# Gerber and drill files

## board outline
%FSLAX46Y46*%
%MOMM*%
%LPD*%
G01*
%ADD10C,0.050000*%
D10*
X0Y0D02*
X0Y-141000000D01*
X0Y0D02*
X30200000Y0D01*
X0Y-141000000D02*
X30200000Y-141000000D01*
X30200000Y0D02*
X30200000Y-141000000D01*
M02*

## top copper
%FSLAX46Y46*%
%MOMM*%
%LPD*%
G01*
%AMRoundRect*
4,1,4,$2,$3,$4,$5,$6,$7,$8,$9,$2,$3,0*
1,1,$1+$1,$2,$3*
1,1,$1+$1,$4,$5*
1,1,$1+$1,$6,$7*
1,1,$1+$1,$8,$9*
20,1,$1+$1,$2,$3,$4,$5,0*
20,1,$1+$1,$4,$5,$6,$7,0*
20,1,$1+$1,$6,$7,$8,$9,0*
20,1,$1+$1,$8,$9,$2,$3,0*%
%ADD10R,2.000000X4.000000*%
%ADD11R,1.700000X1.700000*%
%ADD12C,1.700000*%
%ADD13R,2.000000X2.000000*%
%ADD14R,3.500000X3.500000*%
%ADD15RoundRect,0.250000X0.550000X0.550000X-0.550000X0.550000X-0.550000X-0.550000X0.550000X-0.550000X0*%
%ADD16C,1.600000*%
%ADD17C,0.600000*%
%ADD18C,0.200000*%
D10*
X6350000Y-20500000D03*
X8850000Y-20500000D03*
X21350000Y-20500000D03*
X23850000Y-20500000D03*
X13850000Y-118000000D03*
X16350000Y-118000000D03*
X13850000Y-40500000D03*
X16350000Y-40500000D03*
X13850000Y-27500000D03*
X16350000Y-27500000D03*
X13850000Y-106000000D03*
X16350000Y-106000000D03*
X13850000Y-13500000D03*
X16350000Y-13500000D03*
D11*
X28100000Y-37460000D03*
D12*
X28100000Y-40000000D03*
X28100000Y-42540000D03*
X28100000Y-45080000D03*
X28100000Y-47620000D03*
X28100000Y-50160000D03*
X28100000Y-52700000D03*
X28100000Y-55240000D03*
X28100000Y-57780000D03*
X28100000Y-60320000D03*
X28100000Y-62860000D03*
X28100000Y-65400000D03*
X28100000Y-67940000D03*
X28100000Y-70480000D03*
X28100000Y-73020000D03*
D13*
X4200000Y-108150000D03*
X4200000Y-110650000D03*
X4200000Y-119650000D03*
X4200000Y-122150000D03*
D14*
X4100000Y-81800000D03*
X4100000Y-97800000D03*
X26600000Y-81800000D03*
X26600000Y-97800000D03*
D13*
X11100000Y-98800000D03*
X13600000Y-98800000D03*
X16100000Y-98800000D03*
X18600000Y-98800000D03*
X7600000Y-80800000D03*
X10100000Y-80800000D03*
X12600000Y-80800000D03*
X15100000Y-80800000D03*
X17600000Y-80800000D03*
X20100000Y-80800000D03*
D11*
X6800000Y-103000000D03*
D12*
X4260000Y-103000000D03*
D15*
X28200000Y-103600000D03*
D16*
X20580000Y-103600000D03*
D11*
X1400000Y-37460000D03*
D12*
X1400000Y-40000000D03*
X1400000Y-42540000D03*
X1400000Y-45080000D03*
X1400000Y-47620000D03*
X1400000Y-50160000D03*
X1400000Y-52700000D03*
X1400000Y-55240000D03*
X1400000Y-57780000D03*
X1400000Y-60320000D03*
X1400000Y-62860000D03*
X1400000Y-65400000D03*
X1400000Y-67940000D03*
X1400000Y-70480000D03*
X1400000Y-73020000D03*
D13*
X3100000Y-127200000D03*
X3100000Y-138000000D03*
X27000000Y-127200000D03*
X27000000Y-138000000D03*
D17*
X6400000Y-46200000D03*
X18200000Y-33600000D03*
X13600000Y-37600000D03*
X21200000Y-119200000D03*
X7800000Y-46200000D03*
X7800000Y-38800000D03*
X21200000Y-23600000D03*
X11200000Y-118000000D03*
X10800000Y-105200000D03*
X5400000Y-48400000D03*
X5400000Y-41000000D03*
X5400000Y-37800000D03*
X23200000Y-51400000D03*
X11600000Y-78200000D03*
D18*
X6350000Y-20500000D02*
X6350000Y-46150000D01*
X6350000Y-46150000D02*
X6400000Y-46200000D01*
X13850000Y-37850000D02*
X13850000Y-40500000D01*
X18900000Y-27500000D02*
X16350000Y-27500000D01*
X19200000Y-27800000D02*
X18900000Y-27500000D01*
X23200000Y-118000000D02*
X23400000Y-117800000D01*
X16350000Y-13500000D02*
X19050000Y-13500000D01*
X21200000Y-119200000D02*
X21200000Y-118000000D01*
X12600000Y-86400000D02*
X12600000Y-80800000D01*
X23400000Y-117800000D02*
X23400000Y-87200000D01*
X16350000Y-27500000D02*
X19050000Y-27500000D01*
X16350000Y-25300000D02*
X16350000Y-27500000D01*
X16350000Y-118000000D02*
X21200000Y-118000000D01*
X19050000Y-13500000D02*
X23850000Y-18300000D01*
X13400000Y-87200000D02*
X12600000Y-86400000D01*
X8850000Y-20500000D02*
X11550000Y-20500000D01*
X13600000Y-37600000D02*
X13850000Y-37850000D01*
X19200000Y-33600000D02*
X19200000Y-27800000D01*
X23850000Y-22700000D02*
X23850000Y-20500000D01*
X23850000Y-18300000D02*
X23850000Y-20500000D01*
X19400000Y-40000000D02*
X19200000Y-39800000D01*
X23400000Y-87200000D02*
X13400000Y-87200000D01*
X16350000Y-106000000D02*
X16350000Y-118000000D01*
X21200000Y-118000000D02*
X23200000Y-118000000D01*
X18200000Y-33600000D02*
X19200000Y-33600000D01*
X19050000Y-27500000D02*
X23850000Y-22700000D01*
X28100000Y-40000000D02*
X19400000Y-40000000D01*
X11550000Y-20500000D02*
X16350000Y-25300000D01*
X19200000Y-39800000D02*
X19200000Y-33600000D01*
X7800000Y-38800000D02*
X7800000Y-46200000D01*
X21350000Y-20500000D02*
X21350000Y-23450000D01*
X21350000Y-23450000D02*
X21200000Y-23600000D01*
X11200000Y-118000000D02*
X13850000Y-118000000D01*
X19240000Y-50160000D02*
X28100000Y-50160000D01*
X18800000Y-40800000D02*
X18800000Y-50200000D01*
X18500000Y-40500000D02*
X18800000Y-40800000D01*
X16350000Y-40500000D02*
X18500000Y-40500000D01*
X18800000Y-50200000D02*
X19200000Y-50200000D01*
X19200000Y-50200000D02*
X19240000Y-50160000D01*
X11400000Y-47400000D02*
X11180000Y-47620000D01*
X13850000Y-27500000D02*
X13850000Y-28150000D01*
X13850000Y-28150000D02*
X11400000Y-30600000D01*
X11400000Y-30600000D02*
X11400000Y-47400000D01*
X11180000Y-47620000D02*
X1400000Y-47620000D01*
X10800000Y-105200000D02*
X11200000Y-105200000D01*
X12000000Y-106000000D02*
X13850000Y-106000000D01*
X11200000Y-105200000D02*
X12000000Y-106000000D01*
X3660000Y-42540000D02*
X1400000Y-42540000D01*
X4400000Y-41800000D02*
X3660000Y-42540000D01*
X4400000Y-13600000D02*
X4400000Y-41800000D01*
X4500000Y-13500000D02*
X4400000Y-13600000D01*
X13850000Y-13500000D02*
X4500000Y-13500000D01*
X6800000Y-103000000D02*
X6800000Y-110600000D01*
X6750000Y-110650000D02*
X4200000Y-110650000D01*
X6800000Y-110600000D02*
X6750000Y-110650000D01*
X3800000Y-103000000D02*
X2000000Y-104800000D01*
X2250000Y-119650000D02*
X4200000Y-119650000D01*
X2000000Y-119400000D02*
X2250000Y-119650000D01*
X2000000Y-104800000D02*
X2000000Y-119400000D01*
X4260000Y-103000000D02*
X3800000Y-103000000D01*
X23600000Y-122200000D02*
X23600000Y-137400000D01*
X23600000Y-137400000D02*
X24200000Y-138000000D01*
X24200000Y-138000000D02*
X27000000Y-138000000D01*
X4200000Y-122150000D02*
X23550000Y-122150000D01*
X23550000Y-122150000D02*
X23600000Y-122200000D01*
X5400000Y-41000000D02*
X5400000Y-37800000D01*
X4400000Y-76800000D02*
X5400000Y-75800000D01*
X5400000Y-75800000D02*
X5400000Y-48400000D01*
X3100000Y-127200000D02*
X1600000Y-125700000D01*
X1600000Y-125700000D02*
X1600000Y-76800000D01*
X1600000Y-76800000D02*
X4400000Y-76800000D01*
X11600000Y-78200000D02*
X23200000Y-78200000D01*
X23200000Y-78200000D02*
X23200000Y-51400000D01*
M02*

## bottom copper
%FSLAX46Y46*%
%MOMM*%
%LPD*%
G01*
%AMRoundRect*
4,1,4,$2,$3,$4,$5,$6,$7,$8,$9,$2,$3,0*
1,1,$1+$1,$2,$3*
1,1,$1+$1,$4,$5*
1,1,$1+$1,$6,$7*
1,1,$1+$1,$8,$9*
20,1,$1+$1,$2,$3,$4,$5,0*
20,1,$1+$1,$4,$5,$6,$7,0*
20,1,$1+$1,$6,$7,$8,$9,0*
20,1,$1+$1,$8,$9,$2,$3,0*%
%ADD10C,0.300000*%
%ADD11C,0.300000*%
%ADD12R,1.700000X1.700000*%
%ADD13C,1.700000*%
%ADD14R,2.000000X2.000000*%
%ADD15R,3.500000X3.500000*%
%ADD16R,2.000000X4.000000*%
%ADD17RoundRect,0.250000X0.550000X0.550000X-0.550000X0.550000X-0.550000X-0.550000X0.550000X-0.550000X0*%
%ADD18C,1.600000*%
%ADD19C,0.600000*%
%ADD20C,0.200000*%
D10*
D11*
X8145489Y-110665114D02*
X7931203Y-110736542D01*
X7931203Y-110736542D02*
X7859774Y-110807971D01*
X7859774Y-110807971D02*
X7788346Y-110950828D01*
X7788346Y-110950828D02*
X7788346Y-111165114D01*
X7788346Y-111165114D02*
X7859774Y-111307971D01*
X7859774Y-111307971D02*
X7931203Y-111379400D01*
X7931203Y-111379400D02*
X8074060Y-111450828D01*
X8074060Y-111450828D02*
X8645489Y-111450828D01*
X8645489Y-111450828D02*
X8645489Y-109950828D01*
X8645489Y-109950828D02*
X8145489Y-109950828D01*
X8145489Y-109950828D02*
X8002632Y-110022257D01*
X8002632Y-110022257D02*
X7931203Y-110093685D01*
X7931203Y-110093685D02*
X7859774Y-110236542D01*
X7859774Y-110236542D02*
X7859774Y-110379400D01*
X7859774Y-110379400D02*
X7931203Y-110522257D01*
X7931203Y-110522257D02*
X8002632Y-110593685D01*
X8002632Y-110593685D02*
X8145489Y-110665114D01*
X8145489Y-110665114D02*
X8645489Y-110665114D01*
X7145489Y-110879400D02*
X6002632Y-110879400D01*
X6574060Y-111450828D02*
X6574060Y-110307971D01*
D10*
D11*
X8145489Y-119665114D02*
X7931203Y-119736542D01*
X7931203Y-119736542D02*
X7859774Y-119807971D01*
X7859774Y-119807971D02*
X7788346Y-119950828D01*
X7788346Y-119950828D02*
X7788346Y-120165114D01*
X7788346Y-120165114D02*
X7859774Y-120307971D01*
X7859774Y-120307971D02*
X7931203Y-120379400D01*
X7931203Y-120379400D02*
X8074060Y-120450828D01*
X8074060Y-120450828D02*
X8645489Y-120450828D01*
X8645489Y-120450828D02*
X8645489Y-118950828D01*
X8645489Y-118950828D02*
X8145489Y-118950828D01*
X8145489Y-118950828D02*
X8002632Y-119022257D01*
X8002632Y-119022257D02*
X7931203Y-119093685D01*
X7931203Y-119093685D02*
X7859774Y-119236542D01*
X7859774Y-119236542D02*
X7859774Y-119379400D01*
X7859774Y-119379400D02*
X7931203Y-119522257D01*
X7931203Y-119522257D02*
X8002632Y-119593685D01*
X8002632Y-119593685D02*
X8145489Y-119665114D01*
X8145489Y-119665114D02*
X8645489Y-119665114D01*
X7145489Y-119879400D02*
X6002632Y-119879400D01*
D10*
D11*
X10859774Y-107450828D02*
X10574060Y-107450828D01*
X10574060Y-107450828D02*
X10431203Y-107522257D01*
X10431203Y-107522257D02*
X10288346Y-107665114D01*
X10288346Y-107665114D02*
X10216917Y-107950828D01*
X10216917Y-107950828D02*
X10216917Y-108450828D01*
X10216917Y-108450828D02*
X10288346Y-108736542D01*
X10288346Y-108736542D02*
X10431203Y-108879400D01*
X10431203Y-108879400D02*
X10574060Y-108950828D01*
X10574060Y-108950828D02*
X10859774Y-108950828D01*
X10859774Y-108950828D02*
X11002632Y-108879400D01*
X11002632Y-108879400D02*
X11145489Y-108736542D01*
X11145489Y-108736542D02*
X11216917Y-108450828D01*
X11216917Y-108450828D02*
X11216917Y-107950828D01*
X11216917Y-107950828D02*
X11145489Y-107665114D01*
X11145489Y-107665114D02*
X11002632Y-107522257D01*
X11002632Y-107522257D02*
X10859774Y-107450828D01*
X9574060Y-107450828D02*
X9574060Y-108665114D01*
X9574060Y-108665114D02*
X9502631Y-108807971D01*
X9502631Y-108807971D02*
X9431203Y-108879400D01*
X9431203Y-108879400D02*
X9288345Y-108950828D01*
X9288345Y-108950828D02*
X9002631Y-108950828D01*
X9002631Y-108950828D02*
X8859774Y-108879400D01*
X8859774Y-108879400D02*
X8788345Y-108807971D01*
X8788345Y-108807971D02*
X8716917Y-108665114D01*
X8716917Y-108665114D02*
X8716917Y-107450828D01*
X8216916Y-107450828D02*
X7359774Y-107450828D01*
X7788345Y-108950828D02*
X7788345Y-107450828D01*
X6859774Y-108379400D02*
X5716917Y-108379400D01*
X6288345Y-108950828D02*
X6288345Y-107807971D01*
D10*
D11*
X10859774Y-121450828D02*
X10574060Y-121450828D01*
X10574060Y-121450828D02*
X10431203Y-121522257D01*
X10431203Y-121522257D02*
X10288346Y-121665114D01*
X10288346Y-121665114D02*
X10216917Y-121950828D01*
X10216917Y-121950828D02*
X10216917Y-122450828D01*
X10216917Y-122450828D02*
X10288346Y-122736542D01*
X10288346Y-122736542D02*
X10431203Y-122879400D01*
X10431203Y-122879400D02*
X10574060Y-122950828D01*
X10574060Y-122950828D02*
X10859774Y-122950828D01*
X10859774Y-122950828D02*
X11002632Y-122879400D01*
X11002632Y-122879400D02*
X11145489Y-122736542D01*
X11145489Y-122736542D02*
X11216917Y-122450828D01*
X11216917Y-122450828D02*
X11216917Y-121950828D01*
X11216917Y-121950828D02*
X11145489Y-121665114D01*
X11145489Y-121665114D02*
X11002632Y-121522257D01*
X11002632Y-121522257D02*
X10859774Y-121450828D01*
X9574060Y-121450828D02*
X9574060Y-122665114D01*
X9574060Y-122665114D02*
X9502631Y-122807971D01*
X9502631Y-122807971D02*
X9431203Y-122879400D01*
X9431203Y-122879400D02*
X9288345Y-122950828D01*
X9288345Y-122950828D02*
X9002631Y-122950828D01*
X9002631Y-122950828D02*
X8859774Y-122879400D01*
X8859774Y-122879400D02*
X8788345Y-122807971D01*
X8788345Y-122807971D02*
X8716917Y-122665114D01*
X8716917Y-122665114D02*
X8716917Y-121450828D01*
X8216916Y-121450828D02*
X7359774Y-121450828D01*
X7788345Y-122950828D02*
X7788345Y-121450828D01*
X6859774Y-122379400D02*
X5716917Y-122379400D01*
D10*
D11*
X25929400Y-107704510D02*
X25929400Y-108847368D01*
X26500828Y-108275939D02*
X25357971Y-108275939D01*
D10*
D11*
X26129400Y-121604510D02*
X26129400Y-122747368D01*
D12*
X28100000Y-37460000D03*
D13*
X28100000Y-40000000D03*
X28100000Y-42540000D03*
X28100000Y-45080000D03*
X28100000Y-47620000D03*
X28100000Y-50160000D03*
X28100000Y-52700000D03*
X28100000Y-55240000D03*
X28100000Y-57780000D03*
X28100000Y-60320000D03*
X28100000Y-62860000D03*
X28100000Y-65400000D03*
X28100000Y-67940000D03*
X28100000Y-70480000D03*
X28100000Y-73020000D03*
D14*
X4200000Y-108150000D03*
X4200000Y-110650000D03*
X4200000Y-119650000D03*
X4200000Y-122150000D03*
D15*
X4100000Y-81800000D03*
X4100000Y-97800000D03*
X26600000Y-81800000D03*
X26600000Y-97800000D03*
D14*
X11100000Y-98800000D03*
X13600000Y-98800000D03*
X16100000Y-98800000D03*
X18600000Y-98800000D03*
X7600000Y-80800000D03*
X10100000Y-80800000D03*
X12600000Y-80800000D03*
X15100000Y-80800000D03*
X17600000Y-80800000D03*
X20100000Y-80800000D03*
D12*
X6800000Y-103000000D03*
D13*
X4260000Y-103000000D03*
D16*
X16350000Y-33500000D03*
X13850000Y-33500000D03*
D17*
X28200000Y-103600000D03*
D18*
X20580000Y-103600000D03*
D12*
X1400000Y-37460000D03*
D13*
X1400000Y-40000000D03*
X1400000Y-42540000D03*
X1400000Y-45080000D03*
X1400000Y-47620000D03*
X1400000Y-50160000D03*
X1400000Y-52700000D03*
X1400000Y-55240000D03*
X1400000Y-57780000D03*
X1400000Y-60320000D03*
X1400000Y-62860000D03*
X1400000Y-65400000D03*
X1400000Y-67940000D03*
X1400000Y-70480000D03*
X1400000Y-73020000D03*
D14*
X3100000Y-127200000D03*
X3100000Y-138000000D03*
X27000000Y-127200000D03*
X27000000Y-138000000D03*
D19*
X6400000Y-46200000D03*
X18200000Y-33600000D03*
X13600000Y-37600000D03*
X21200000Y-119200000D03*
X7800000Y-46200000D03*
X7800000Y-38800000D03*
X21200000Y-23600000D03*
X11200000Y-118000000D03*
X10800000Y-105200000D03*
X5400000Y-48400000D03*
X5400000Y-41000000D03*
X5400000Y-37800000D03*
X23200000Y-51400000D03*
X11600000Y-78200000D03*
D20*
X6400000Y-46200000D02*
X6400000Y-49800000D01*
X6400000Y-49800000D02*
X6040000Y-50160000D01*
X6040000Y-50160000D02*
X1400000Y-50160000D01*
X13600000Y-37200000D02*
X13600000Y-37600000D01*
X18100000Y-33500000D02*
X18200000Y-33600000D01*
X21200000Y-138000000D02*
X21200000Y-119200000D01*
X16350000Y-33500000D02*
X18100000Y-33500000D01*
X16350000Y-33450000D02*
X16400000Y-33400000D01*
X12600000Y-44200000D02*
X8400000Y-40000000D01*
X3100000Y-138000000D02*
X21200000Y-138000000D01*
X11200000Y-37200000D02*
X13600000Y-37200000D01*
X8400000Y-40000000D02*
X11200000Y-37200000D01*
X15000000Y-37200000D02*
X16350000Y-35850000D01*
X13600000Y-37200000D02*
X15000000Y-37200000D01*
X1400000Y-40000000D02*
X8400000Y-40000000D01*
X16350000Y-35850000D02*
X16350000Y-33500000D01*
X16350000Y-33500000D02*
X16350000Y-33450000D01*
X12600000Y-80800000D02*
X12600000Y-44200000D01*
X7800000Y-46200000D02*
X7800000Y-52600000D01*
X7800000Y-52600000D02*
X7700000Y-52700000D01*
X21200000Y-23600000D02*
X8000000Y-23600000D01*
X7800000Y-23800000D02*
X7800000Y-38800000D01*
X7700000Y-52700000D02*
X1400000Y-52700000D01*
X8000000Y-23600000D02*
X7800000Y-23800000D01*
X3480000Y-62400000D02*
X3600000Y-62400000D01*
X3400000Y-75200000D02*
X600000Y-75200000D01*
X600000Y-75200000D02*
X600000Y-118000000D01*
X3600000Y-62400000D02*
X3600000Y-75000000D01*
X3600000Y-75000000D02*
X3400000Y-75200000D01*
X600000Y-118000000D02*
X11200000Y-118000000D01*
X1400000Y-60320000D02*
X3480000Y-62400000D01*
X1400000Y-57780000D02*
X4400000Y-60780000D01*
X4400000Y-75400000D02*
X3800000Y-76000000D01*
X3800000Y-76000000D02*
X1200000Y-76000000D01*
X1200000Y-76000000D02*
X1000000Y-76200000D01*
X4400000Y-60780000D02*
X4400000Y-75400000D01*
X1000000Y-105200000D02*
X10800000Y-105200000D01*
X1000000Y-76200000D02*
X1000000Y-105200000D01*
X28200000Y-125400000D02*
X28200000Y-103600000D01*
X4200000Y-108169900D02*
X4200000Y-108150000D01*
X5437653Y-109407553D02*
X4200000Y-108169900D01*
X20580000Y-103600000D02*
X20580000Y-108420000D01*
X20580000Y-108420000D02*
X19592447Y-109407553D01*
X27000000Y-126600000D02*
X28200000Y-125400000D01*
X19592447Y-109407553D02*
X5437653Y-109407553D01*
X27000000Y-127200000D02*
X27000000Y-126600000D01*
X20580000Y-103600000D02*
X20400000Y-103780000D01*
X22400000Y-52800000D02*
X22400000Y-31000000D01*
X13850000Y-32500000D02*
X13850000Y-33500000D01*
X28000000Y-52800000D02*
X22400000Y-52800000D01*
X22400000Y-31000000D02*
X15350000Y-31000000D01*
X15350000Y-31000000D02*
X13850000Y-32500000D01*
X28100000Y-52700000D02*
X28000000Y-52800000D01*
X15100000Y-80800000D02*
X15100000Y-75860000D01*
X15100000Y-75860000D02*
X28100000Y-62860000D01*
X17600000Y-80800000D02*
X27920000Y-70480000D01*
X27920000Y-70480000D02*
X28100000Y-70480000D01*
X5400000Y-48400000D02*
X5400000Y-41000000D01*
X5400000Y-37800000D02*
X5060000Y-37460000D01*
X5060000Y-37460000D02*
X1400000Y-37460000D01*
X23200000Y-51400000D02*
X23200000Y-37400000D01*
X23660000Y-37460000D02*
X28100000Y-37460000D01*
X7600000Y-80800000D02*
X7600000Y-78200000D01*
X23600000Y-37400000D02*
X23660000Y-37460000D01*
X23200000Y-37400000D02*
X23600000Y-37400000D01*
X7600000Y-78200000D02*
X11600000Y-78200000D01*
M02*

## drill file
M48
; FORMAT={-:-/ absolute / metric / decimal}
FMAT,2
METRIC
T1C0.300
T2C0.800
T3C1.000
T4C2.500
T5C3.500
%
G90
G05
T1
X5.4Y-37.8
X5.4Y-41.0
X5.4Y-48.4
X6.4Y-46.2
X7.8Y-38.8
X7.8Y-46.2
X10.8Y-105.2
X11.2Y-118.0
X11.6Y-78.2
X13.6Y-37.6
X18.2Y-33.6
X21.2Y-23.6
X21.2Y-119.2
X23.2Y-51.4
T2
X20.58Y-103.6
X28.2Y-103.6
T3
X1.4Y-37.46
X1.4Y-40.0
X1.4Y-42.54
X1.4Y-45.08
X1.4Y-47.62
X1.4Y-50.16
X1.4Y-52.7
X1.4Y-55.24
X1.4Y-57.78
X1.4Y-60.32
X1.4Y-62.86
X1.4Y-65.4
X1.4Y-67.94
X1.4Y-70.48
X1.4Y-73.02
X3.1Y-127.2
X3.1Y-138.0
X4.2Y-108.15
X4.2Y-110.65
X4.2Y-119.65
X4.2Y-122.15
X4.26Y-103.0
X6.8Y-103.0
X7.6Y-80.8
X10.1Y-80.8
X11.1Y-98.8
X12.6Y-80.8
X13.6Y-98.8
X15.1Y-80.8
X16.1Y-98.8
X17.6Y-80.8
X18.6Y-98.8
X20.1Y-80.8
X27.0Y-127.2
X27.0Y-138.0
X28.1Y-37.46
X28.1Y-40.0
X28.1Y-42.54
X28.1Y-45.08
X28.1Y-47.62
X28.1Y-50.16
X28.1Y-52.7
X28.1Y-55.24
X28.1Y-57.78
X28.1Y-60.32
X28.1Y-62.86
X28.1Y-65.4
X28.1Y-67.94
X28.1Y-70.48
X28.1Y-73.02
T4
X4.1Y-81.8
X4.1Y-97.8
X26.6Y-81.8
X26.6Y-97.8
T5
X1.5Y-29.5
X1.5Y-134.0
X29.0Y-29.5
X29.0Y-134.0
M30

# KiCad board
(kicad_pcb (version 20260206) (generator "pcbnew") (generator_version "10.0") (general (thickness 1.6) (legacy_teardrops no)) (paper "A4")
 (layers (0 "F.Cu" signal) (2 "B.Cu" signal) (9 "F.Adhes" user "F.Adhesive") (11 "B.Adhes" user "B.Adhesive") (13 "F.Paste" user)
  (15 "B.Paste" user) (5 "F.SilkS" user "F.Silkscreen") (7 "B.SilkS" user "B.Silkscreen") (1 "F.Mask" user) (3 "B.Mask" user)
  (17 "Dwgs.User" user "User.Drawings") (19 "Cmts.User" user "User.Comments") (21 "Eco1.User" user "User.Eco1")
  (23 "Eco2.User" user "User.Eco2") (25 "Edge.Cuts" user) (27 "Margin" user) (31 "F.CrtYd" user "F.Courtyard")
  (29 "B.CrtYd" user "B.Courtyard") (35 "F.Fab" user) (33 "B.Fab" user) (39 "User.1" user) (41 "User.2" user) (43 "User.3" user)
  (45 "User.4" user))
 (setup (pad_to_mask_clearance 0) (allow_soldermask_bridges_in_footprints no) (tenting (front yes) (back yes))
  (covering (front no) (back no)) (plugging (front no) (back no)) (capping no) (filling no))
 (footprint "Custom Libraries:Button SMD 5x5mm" (layer "F.Cu") (at 4.85 18)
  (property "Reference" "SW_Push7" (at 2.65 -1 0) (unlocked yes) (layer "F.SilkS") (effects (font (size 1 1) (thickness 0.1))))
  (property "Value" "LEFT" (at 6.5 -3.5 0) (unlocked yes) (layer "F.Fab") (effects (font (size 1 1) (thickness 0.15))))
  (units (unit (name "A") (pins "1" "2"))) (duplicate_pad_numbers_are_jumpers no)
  (pad "1" smd rect (at 1.5 2.5 180) (size 2 4) (layers "F.Cu" "F.Mask" "F.Paste") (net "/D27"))
  (pad "2" smd rect (at 4 2.5 180) (size 2 4) (layers "F.Cu" "F.Mask" "F.Paste") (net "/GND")))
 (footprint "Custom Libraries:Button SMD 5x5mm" (layer "F.Cu") (at 19.85 18)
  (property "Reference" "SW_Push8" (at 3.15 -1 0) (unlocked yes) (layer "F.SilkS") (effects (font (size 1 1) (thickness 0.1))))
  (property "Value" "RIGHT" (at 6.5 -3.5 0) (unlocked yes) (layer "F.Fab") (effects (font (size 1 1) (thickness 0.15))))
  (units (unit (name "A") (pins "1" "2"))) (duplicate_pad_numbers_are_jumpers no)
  (pad "1" smd rect (at 1.5 2.5 180) (size 2 4) (layers "F.Cu" "F.Mask" "F.Paste") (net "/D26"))
  (pad "2" smd rect (at 4 2.5 180) (size 2 4) (layers "F.Cu" "F.Mask" "F.Paste") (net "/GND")))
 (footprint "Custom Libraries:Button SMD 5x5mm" (layer "F.Cu") (at 12.35 115.5)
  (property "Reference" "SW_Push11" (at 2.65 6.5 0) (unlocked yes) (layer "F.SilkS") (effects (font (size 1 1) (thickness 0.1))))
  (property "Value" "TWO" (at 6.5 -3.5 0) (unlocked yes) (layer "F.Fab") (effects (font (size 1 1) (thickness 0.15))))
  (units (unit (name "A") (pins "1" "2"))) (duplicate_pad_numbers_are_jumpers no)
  (pad "1" smd rect (at 1.5 2.5 180) (size 2 4) (layers "F.Cu" "F.Mask" "F.Paste") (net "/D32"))
  (pad "2" smd rect (at 4 2.5 180) (size 2 4) (layers "F.Cu" "F.Mask" "F.Paste") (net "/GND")))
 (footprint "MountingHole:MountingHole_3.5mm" (layer "F.Cu") (at 29 134)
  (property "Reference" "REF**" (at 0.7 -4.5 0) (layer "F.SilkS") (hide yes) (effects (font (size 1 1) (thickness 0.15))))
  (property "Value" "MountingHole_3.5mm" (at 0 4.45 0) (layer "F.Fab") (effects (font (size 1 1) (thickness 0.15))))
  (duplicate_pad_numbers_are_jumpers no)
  (pad "" np_thru_hole circle (at 0 0) (size 3.5 3.5) (drill 3.5) (layers "*.Cu" "*.Mask")))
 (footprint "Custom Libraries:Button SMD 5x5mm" (layer "F.Cu") (at 12.35 38)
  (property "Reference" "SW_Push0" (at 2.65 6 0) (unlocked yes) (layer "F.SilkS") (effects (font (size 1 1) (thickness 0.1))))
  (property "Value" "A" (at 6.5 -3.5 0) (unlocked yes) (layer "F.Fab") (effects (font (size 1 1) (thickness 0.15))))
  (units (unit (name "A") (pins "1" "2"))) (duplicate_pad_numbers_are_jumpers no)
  (pad "1" smd rect (at 1.5 2.5 180) (size 2 4) (layers "F.Cu" "F.Mask" "F.Paste") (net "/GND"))
  (pad "2" smd rect (at 4 2.5 180) (size 2 4) (layers "F.Cu" "F.Mask" "F.Paste") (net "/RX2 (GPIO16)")))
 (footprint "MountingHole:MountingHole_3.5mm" (layer "F.Cu") (at 1.5 134)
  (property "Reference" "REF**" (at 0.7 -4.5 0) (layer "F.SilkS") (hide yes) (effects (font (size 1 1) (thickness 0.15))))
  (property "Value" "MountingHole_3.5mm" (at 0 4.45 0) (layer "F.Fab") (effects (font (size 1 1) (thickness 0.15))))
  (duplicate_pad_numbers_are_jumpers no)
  (pad "" np_thru_hole circle (at 0 0) (size 3.5 3.5) (drill 3.5) (layers "*.Cu" "*.Mask")))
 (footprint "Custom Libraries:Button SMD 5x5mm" (layer "F.Cu") (at 12.35 25)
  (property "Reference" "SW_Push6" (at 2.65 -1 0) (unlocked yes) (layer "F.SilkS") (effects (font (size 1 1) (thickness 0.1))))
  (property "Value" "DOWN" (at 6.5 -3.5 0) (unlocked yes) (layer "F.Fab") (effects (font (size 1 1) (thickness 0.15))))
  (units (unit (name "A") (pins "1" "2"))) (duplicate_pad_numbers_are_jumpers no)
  (pad "1" smd rect (at 1.5 2.5 180) (size 2 4) (layers "F.Cu" "F.Mask" "F.Paste") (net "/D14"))
  (pad "2" smd rect (at 4 2.5 180) (size 2 4) (layers "F.Cu" "F.Mask" "F.Paste") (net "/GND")))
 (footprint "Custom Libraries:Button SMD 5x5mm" (layer "F.Cu") (at 12.35 103.5)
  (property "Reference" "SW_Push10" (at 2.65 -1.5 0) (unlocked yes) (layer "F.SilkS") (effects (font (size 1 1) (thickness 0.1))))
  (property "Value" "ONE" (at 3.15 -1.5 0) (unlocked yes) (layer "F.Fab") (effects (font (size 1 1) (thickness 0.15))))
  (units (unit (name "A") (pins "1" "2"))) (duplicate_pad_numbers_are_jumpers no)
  (pad "1" smd rect (at 1.5 2.5 180) (size 2 4) (layers "F.Cu" "F.Mask" "F.Paste") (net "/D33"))
  (pad "2" smd rect (at 4 2.5 180) (size 2 4) (layers "F.Cu" "F.Mask" "F.Paste") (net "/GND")))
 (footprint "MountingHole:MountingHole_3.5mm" (layer "F.Cu") (at 1.5 29.5)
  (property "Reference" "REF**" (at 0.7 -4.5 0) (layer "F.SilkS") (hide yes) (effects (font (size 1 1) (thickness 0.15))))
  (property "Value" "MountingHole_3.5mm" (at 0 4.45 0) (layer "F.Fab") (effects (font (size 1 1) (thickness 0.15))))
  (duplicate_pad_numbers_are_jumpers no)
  (pad "" np_thru_hole circle (at 0 0) (size 3.5 3.5) (drill 3.5) (layers "*.Cu" "*.Mask")))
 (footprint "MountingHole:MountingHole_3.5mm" (layer "F.Cu") (at 29 29.5)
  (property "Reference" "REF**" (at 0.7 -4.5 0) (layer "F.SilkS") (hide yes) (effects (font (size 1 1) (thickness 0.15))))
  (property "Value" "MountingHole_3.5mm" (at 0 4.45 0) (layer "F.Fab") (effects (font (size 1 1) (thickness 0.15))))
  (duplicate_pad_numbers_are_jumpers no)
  (pad "" np_thru_hole circle (at 0 0) (size 3.5 3.5) (drill 3.5) (layers "*.Cu" "*.Mask")))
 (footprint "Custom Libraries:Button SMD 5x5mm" (layer "F.Cu") (at 12.35 11)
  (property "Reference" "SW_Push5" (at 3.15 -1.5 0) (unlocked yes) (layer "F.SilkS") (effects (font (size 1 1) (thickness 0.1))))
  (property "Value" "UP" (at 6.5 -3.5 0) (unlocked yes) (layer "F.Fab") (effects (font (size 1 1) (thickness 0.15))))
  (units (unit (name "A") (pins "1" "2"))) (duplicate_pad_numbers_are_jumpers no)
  (pad "1" smd rect (at 1.5 2.5 180) (size 2 4) (layers "F.Cu" "F.Mask" "F.Paste") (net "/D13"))
  (pad "2" smd rect (at 4 2.5 180) (size 2 4) (layers "F.Cu" "F.Mask" "F.Paste") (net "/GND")))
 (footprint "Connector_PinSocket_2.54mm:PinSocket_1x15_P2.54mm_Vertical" (layer "B.Cu") (at 28.1 37.46 180)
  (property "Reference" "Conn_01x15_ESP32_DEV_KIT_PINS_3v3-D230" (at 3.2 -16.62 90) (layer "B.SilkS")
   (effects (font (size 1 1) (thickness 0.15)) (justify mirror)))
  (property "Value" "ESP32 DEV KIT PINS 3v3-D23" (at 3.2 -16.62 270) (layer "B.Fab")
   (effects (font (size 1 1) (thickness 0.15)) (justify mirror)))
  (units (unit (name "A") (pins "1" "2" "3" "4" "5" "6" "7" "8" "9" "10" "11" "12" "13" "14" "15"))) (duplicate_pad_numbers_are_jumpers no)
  (pad "1" thru_hole rect (at 0 0 180) (size 1.7 1.7) (drill 1) (layers "*.Cu" "*.Mask") (remove_unused_layers no) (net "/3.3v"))
  (pad "2" thru_hole circle (at 0 -2.54 180) (size 1.7 1.7) (drill 1) (layers "*.Cu" "*.Mask") (remove_unused_layers no) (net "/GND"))
  (pad "3" thru_hole circle (at 0 -5.08 180) (size 1.7 1.7) (drill 1) (layers "*.Cu" "*.Mask") (remove_unused_layers no)
   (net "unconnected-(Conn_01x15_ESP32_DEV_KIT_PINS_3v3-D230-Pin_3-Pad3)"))
  (pad "4" thru_hole circle (at 0 -7.62 180) (size 1.7 1.7) (drill 1) (layers "*.Cu" "*.Mask") (remove_unused_layers no)
   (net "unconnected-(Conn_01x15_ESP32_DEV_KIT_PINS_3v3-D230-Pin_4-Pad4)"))
  (pad "5" thru_hole circle (at 0 -10.16 180) (size 1.7 1.7) (drill 1) (layers "*.Cu" "*.Mask") (remove_unused_layers no)
   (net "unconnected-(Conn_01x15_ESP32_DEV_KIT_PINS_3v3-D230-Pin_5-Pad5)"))
  (pad "6" thru_hole circle (at 0 -12.7 180) (size 1.7 1.7) (drill 1) (layers "*.Cu" "*.Mask") (remove_unused_layers no)
   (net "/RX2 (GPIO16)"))
  (pad "7" thru_hole circle (at 0 -15.24 180) (size 1.7 1.7) (drill 1) (layers "*.Cu" "*.Mask") (remove_unused_layers no)
   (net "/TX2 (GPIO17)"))
  (pad "8" thru_hole circle (at 0 -17.78 180) (size 1.7 1.7) (drill 1) (layers "*.Cu" "*.Mask") (remove_unused_layers no)
   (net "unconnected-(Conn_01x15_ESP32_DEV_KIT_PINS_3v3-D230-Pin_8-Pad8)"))
  (pad "9" thru_hole circle (at 0 -20.32 180) (size 1.7 1.7) (drill 1) (layers "*.Cu" "*.Mask") (remove_unused_layers no)
   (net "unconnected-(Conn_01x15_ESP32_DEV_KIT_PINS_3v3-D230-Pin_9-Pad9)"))
  (pad "10" thru_hole circle (at 0 -22.86 180) (size 1.7 1.7) (drill 1) (layers "*.Cu" "*.Mask") (remove_unused_layers no)
   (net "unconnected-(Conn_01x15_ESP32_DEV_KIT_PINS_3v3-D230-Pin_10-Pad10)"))
  (pad "11" thru_hole circle (at 0 -25.4 180) (size 1.7 1.7) (drill 1) (layers "*.Cu" "*.Mask") (remove_unused_layers no) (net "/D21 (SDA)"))
  (pad "12" thru_hole circle (at 0 -27.94 180) (size 1.7 1.7) (drill 1) (layers "*.Cu" "*.Mask") (remove_unused_layers no)
   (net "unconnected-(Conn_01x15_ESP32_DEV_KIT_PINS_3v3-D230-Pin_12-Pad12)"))
  (pad "13" thru_hole circle (at 0 -30.48 180) (size 1.7 1.7) (drill 1) (layers "*.Cu" "*.Mask") (remove_unused_layers no)
   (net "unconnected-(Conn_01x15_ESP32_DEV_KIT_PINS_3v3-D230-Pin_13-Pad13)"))
  (pad "14" thru_hole circle (at 0 -33.02 180) (size 1.7 1.7) (drill 1) (layers "*.Cu" "*.Mask") (remove_unused_layers no)
   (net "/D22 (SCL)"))
  (pad "15" thru_hole circle (at 0 -35.56 180) (size 1.7 1.7) (drill 1) (layers "*.Cu" "*.Mask") (remove_unused_layers no)
   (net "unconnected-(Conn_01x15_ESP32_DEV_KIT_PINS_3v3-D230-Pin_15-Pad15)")))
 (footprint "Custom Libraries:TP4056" (layer "B.Cu") (at 1.2 106.65 -90)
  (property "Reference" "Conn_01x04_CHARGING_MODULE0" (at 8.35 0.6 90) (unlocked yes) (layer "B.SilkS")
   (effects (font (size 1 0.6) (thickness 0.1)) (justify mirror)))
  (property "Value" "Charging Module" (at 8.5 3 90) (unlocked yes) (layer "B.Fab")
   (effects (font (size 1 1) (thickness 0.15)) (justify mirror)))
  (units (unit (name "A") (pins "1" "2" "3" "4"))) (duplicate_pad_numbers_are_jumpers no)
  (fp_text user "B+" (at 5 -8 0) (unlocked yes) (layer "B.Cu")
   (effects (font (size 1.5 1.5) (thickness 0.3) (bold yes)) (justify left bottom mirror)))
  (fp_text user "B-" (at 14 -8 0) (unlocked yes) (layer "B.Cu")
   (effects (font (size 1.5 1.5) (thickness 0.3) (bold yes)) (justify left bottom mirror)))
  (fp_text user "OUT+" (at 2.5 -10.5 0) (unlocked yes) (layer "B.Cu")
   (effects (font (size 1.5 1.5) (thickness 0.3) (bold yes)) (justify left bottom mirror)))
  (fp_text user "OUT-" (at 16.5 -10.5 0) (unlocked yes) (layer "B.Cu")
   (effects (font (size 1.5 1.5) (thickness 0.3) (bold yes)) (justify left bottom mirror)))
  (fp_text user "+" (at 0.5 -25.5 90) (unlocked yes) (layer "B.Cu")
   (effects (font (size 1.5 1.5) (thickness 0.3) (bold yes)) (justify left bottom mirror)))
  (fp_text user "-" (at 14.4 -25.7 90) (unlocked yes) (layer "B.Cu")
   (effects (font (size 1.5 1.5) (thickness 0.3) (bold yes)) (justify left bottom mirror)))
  (pad "1" thru_hole rect (at 1.5 -3 270) (size 2 2) (drill 1) (layers "*.Cu" "*.Mask") (remove_unused_layers no) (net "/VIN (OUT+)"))
  (pad "2" thru_hole rect (at 4 -3 270) (size 2 2) (drill 1) (layers "*.Cu" "*.Mask") (remove_unused_layers no) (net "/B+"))
  (pad "3" thru_hole rect (at 13 -3 270) (size 2 2) (drill 1) (layers "*.Cu" "*.Mask") (remove_unused_layers no) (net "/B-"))
  (pad "4" thru_hole rect (at 15.5 -3 270) (size 2 2) (drill 1) (layers "*.Cu" "*.Mask") (remove_unused_layers no) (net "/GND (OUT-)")))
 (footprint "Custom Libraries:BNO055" (layer "B.Cu") (at 2.1 99.8)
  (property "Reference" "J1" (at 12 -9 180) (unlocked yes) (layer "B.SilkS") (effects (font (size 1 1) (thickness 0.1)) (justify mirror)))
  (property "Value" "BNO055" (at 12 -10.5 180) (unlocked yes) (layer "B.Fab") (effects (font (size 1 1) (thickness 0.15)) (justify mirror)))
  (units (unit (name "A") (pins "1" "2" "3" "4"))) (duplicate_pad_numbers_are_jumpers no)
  (pad "" np_thru_hole rect (at 2 -18) (size 3.5 3.5) (drill 2.5) (layers "*.Cu" "*.Mask"))
  (pad "" np_thru_hole rect (at 2 -2) (size 3.5 3.5) (drill 2.5) (layers "*.Cu" "*.Mask"))
  (pad "" np_thru_hole rect (at 24.5 -18) (size 3.5 3.5) (drill 2.5) (layers "*.Cu" "*.Mask"))
  (pad "" np_thru_hole rect (at 24.5 -2) (size 3.5 3.5) (drill 2.5) (layers "*.Cu" "*.Mask"))
  (pad "1" thru_hole rect (at 9 -1) (size 2 2) (drill 1) (layers "*.Cu" "*.Mask") (remove_unused_layers no))
  (pad "2" thru_hole rect (at 11.5 -1) (size 2 2) (drill 1) (layers "*.Cu" "*.Mask") (remove_unused_layers no))
  (pad "3" thru_hole rect (at 14 -1) (size 2 2) (drill 1) (layers "*.Cu" "*.Mask") (remove_unused_layers no))
  (pad "4" thru_hole rect (at 16.5 -1) (size 2 2) (drill 1) (layers "*.Cu" "*.Mask") (remove_unused_layers no))
  (pad "5" thru_hole rect (at 5.5 -19) (size 2 2) (drill 1) (layers "*.Cu" "*.Mask") (remove_unused_layers no) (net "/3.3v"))
  (pad "6" thru_hole rect (at 8 -19) (size 2 2) (drill 1) (layers "*.Cu" "*.Mask") (remove_unused_layers no))
  (pad "7" thru_hole rect (at 10.5 -19) (size 2 2) (drill 1) (layers "*.Cu" "*.Mask") (remove_unused_layers no) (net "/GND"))
  (pad "8" thru_hole rect (at 13 -19) (size 2 2) (drill 1) (layers "*.Cu" "*.Mask") (remove_unused_layers no) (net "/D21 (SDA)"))
  (pad "9" thru_hole rect (at 15.5 -19) (size 2 2) (drill 1) (layers "*.Cu" "*.Mask") (remove_unused_layers no) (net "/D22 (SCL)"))
  (pad "10" thru_hole rect (at 18 -19) (size 2 2) (drill 1) (layers "*.Cu" "*.Mask") (remove_unused_layers no)))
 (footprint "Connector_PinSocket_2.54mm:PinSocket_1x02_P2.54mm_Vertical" (layer "B.Cu") (at 6.8 103 90)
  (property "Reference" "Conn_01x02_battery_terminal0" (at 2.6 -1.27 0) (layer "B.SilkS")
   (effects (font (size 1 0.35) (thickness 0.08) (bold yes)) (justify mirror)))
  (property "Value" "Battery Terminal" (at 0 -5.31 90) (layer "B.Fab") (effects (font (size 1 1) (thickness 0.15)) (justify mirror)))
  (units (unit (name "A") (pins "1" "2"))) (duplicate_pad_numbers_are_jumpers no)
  (pad "1" thru_hole rect (at 0 0 90) (size 1.7 1.7) (drill 1) (layers "*.Cu" "*.Mask") (remove_unused_layers no) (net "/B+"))
  (pad "2" thru_hole circle (at 0 -2.54 90) (size 1.7 1.7) (drill 1) (layers "*.Cu" "*.Mask") (remove_unused_layers no) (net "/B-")))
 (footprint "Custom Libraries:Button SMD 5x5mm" (layer "B.Cu") (at 17.85 31 180)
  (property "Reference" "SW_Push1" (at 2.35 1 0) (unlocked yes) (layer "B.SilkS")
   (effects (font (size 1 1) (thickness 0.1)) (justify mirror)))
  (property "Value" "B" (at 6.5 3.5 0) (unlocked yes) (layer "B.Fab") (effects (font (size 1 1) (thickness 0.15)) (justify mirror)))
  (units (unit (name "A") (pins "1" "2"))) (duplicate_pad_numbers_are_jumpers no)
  (pad "1" smd rect (at 1.5 -2.5) (size 2 4) (layers "B.Cu" "B.Mask" "B.Paste") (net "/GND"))
  (pad "2" smd rect (at 4 -2.5) (size 2 4) (layers "B.Cu" "B.Mask" "B.Paste") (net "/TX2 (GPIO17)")))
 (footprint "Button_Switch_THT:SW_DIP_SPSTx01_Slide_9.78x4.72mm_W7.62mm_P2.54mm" (layer "B.Cu") (at 28.2 103.6 180)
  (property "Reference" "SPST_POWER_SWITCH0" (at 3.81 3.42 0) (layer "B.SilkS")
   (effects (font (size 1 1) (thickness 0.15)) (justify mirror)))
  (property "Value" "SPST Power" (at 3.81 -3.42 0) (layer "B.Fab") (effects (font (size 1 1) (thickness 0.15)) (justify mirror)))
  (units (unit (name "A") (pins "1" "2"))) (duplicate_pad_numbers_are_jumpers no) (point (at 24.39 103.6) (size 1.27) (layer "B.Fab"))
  (pad "1" thru_hole roundrect (at 0 0 180) (size 1.6 1.6) (drill 0.8) (layers "*.Cu" "*.Mask") (remove_unused_layers no)
   (roundrect_rratio 0.15625) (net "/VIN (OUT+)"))
  (pad "2" thru_hole circle (at 7.62 0 180) (size 1.6 1.6) (drill 0.8) (layers "*.Cu" "*.Mask") (remove_unused_layers no)
   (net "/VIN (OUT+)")))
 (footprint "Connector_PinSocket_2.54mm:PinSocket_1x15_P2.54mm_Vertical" (layer "B.Cu") (at 1.4 37.46 180)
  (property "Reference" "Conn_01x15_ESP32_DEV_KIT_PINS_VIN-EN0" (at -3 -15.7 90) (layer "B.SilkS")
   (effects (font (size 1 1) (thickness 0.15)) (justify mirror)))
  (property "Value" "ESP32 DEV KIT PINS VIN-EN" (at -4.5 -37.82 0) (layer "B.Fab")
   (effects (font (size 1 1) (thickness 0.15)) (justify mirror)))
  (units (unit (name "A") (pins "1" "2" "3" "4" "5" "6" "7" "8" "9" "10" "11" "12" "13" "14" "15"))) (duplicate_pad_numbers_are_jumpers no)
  (pad "1" thru_hole rect (at 0 0 180) (size 1.7 1.7) (drill 1) (layers "*.Cu" "*.Mask") (remove_unused_layers no) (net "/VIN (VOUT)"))
  (pad "2" thru_hole circle (at 0 -2.54 180) (size 1.7 1.7) (drill 1) (layers "*.Cu" "*.Mask") (remove_unused_layers no) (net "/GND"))
  (pad "3" thru_hole circle (at 0 -5.08 180) (size 1.7 1.7) (drill 1) (layers "*.Cu" "*.Mask") (remove_unused_layers no) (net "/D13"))
  (pad "4" thru_hole circle (at 0 -7.62 180) (size 1.7 1.7) (drill 1) (layers "*.Cu" "*.Mask") (remove_unused_layers no)
   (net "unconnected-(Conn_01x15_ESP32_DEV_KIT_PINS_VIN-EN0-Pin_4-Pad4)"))
  (pad "5" thru_hole circle (at 0 -10.16 180) (size 1.7 1.7) (drill 1) (layers "*.Cu" "*.Mask") (remove_unused_layers no) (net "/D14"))
  (pad "6" thru_hole circle (at 0 -12.7 180) (size 1.7 1.7) (drill 1) (layers "*.Cu" "*.Mask") (remove_unused_layers no) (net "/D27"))
  (pad "7" thru_hole circle (at 0 -15.24 180) (size 1.7 1.7) (drill 1) (layers "*.Cu" "*.Mask") (remove_unused_layers no) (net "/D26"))
  (pad "8" thru_hole circle (at 0 -17.78 180) (size 1.7 1.7) (drill 1) (layers "*.Cu" "*.Mask") (remove_unused_layers no)
   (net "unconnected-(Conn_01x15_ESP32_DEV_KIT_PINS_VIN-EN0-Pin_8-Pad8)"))
  (pad "9" thru_hole circle (at 0 -20.32 180) (size 1.7 1.7) (drill 1) (layers "*.Cu" "*.Mask") (remove_unused_layers no) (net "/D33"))
  (pad "10" thru_hole circle (at 0 -22.86 180) (size 1.7 1.7) (drill 1) (layers "*.Cu" "*.Mask") (remove_unused_layers no) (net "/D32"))
  (pad "11" thru_hole circle (at 0 -25.4 180) (size 1.7 1.7) (drill 1) (layers "*.Cu" "*.Mask") (remove_unused_layers no)
   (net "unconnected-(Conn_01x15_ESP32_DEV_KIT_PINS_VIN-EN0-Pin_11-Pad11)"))
  (pad "12" thru_hole circle (at 0 -27.94 180) (size 1.7 1.7) (drill 1) (layers "*.Cu" "*.Mask") (remove_unused_layers no)
   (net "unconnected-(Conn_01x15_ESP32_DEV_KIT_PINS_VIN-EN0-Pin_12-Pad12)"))
  (pad "13" thru_hole circle (at 0 -30.48 180) (size 1.7 1.7) (drill 1) (layers "*.Cu" "*.Mask") (remove_unused_layers no)
   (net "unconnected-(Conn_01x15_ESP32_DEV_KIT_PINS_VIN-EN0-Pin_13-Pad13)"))
  (pad "14" thru_hole circle (at 0 -33.02 180) (size 1.7 1.7) (drill 1) (layers "*.Cu" "*.Mask") (remove_unused_layers no)
   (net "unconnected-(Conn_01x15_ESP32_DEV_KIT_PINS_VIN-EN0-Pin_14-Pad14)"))
  (pad "15" thru_hole circle (at 0 -35.56 180) (size 1.7 1.7) (drill 1) (layers "*.Cu" "*.Mask") (remove_unused_layers no)
   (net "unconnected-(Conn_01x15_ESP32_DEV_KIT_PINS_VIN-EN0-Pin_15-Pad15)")))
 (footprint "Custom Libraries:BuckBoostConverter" (layer "B.Cu") (at 2.1 126.2 -90)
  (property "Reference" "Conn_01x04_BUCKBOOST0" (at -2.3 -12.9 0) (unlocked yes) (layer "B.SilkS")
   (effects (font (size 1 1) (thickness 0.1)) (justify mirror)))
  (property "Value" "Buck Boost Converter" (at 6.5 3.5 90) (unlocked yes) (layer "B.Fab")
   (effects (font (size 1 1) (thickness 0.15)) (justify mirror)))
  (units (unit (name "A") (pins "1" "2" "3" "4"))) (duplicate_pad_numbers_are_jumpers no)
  (pad "1" thru_hole rect (at 1 -1 270) (size 2 2) (drill 1) (layers "*.Cu" "*.Mask") (remove_unused_layers no) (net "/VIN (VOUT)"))
  (pad "2" thru_hole rect (at 11.8 -1 270) (size 2 2) (drill 1) (layers "*.Cu" "*.Mask") (remove_unused_layers no) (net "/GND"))
  (pad "3" thru_hole rect (at 1 -24.9 270) (size 2 2) (drill 1) (layers "*.Cu" "*.Mask") (remove_unused_layers no) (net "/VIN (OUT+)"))
  (pad "4" thru_hole rect (at 11.8 -24.9 270) (size 2 2) (drill 1) (layers "*.Cu" "*.Mask") (remove_unused_layers no) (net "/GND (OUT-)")))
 (gr_line (start 0 0) (end 0 141) (stroke (width 0.05) (type solid)) (layer "Edge.Cuts"))
 (gr_line (start 0 0) (end 30.2 0) (stroke (width 0.05) (type solid)) (layer "Edge.Cuts"))
 (gr_line (start 0 141) (end 30.2 141) (stroke (width 0.05) (type solid)) (layer "Edge.Cuts"))
 (gr_line (start 30.2 0) (end 30.2 141) (stroke (width 0.05) (type solid)) (layer "Edge.Cuts"))
 (segment (start 6.35 20.5) (end 6.35 46.15) (width 0.2) (layer "F.Cu") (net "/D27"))
 (segment (start 6.35 46.15) (end 6.4 46.2) (width 0.2) (layer "F.Cu") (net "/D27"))
 (via (at 6.4 46.2) (size 0.6) (drill 0.3) (layers "F.Cu" "B.Cu") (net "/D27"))
 (segment (start 6.4 46.2) (end 6.4 49.8) (width 0.2) (layer "B.Cu") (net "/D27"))
 (segment (start 6.4 49.8) (end 6.04 50.16) (width 0.2) (layer "B.Cu") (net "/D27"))
 (segment (start 6.04 50.16) (end 1.4 50.16) (width 0.2) (layer "B.Cu") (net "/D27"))
 (segment (start 13.85 37.85) (end 13.85 40.5) (width 0.2) (layer "F.Cu") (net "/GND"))
 (segment (start 18.9 27.5) (end 16.35 27.5) (width 0.2) (layer "F.Cu") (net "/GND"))
 (segment (start 19.2 27.8) (end 18.9 27.5) (width 0.2) (layer "F.Cu") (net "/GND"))
 (segment (start 23.2 118) (end 23.4 117.8) (width 0.2) (layer "F.Cu") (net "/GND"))
 (segment (start 16.35 13.5) (end 19.05 13.5) (width 0.2) (layer "F.Cu") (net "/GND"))
 (segment (start 21.2 119.2) (end 21.2 118) (width 0.2) (layer "F.Cu") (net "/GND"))
 (segment (start 12.6 86.4) (end 12.6 80.8) (width 0.2) (layer "F.Cu") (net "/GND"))
 (segment (start 23.4 117.8) (end 23.4 87.2) (width 0.2) (layer "F.Cu") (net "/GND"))
 (segment (start 16.35 27.5) (end 19.05 27.5) (width 0.2) (layer "F.Cu") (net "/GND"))
 (segment (start 16.35 25.3) (end 16.35 27.5) (width 0.2) (layer "F.Cu") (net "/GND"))
 (segment (start 16.35 118) (end 21.2 118) (width 0.2) (layer "F.Cu") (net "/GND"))
 (segment (start 19.05 13.5) (end 23.85 18.3) (width 0.2) (layer "F.Cu") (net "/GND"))
 (segment (start 13.4 87.2) (end 12.6 86.4) (width 0.2) (layer "F.Cu") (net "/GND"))
 (segment (start 8.85 20.5) (end 11.55 20.5) (width 0.2) (layer "F.Cu") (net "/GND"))
 (segment (start 13.6 37.6) (end 13.85 37.85) (width 0.2) (layer "F.Cu") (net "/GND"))
 (segment (start 19.2 33.6) (end 19.2 27.8) (width 0.2) (layer "F.Cu") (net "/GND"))
 (segment (start 23.85 22.7) (end 23.85 20.5) (width 0.2) (layer "F.Cu") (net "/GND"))
 (segment (start 23.85 18.3) (end 23.85 20.5) (width 0.2) (layer "F.Cu") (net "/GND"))
 (segment (start 19.4 40) (end 19.2 39.8) (width 0.2) (layer "F.Cu") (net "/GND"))
 (segment (start 23.4 87.2) (end 13.4 87.2) (width 0.2) (layer "F.Cu") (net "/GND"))
 (segment (start 16.35 106) (end 16.35 118) (width 0.2) (layer "F.Cu") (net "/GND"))
 (segment (start 21.2 118) (end 23.2 118) (width 0.2) (layer "F.Cu") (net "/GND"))
 (segment (start 18.2 33.6) (end 19.2 33.6) (width 0.2) (layer "F.Cu") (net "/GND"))
 (segment (start 19.05 27.5) (end 23.85 22.7) (width 0.2) (layer "F.Cu") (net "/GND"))
 (segment (start 28.1 40) (end 19.4 40) (width 0.2) (layer "F.Cu") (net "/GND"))
 (segment (start 11.55 20.5) (end 16.35 25.3) (width 0.2) (layer "F.Cu") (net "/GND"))
 (segment (start 19.2 39.8) (end 19.2 33.6) (width 0.2) (layer "F.Cu") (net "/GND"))
 (via (at 18.2 33.6) (size 0.6) (drill 0.3) (layers "F.Cu" "B.Cu") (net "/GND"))
 (via (at 13.6 37.6) (size 0.6) (drill 0.3) (layers "F.Cu" "B.Cu") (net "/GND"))
 (via (at 21.2 119.2) (size 0.6) (drill 0.3) (layers "F.Cu" "B.Cu") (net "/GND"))
 (segment (start 13.6 37.2) (end 13.6 37.6) (width 0.2) (layer "B.Cu") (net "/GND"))
 (segment (start 18.1 33.5) (end 18.2 33.6) (width 0.2) (layer "B.Cu") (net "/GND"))
 (segment (start 21.2 138) (end 21.2 119.2) (width 0.2) (layer "B.Cu") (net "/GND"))
 (segment (start 16.35 33.5) (end 18.1 33.5) (width 0.2) (layer "B.Cu") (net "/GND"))
 (segment (start 16.35 33.45) (end 16.4 33.4) (width 0.2) (layer "B.Cu") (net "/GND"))
 (segment (start 12.6 44.2) (end 8.4 40) (width 0.2) (layer "B.Cu") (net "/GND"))
 (segment (start 3.1 138) (end 21.2 138) (width 0.2) (layer "B.Cu") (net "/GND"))
 (segment (start 11.2 37.2) (end 13.6 37.2) (width 0.2) (layer "B.Cu") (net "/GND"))
 (segment (start 8.4 40) (end 11.2 37.2) (width 0.2) (layer "B.Cu") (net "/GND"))
 (segment (start 15 37.2) (end 16.35 35.85) (width 0.2) (layer "B.Cu") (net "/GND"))
 (segment (start 13.6 37.2) (end 15 37.2) (width 0.2) (layer "B.Cu") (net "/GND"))
 (segment (start 1.4 40) (end 8.4 40) (width 0.2) (layer "B.Cu") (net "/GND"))
 (segment (start 16.35 35.85) (end 16.35 33.5) (width 0.2) (layer "B.Cu") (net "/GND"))
 (segment (start 16.35 33.5) (end 16.35 33.45) (width 0.2) (layer "B.Cu") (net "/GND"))
 (segment (start 12.6 80.8) (end 12.6 44.2) (width 0.2) (layer "B.Cu") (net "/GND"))
 (segment (start 7.8 38.8) (end 7.8 46.2) (width 0.2) (layer "F.Cu") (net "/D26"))
 (segment (start 21.35 20.5) (end 21.35 23.45) (width 0.2) (layer "F.Cu") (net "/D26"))
 (segment (start 21.35 23.45) (end 21.2 23.6) (width 0.2) (layer "F.Cu") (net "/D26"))
 (via (at 7.8 46.2) (size 0.6) (drill 0.3) (layers "F.Cu" "B.Cu") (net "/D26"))
 (via (at 7.8 38.8) (size 0.6) (drill 0.3) (layers "F.Cu" "B.Cu") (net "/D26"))
 (via (at 21.2 23.6) (size 0.6) (drill 0.3) (layers "F.Cu" "B.Cu") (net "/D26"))
 (segment (start 7.8 46.2) (end 7.8 52.6) (width 0.2) (layer "B.Cu") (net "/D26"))
 (segment (start 7.8 52.6) (end 7.7 52.7) (width 0.2) (layer "B.Cu") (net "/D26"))
 (segment (start 21.2 23.6) (end 8 23.6) (width 0.2) (layer "B.Cu") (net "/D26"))
 (segment (start 7.8 23.8) (end 7.8 38.8) (width 0.2) (layer "B.Cu") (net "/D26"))
 (segment (start 7.7 52.7) (end 1.4 52.7) (width 0.2) (layer "B.Cu") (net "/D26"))
 (segment (start 8 23.6) (end 7.8 23.8) (width 0.2) (layer "B.Cu") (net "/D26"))
 (segment (start 11.2 118) (end 13.85 118) (width 0.2) (layer "F.Cu") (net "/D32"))
 (via (at 11.2 118) (size 0.6) (drill 0.3) (layers "F.Cu" "B.Cu") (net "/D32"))
 (segment (start 3.48 62.4) (end 3.6 62.4) (width 0.2) (layer "B.Cu") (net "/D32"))
 (segment (start 3.4 75.2) (end 0.6 75.2) (width 0.2) (layer "B.Cu") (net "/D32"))
 (segment (start 0.6 75.2) (end 0.6 118) (width 0.2) (layer "B.Cu") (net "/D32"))
 (segment (start 3.6 62.4) (end 3.6 75) (width 0.2) (layer "B.Cu") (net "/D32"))
 (segment (start 3.6 75) (end 3.4 75.2) (width 0.2) (layer "B.Cu") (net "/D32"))
 (segment (start 0.6 118) (end 11.2 118) (width 0.2) (layer "B.Cu") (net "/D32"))
 (segment (start 1.4 60.32) (end 3.48 62.4) (width 0.2) (layer "B.Cu") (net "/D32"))
 (segment (start 19.24 50.16) (end 28.1 50.16) (width 0.2) (layer "F.Cu") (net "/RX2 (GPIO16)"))
 (segment (start 18.8 40.8) (end 18.8 50.2) (width 0.2) (layer "F.Cu") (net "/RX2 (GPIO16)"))
 (segment (start 18.5 40.5) (end 18.8 40.8) (width 0.2) (layer "F.Cu") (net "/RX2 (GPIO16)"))
 (segment (start 16.35 40.5) (end 18.5 40.5) (width 0.2) (layer "F.Cu") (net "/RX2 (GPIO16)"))
 (segment (start 18.8 50.2) (end 19.2 50.2) (width 0.2) (layer "F.Cu") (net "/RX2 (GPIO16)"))
 (segment (start 19.2 50.2) (end 19.24 50.16) (width 0.2) (layer "F.Cu") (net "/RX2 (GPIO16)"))
 (segment (start 11.4 47.4) (end 11.18 47.62) (width 0.2) (layer "F.Cu") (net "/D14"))
 (segment (start 13.85 27.5) (end 13.85 28.15) (width 0.2) (layer "F.Cu") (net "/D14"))
 (segment (start 13.85 28.15) (end 11.4 30.6) (width 0.2) (layer "F.Cu") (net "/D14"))
 (segment (start 11.4 30.6) (end 11.4 47.4) (width 0.2) (layer "F.Cu") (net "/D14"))
 (segment (start 11.18 47.62) (end 1.4 47.62) (width 0.2) (layer "F.Cu") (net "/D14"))
 (segment (start 10.8 105.2) (end 11.2 105.2) (width 0.2) (layer "F.Cu") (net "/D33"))
 (segment (start 12 106) (end 13.85 106) (width 0.2) (layer "F.Cu") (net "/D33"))
 (segment (start 11.2 105.2) (end 12 106) (width 0.2) (layer "F.Cu") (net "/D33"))
 (via (at 10.8 105.2) (size 0.6) (drill 0.3) (layers "F.Cu" "B.Cu") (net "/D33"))
 (segment (start 1.4 57.78) (end 4.4 60.78) (width 0.2) (layer "B.Cu") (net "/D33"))
 (segment (start 4.4 75.4) (end 3.8 76) (width 0.2) (layer "B.Cu") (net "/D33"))
 (segment (start 3.8 76) (end 1.2 76) (width 0.2) (layer "B.Cu") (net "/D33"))
 (segment (start 1.2 76) (end 1 76.2) (width 0.2) (layer "B.Cu") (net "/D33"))
 (segment (start 4.4 60.78) (end 4.4 75.4) (width 0.2) (layer "B.Cu") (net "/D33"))
 (segment (start 1 105.2) (end 10.8 105.2) (width 0.2) (layer "B.Cu") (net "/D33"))
 (segment (start 1 76.2) (end 1 105.2) (width 0.2) (layer "B.Cu") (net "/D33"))
 (segment (start 28.2 125.4) (end 28.2 103.6) (width 0.2) (layer "B.Cu") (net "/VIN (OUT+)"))
 (segment (start 4.2 108.1699) (end 4.2 108.15) (width 0.2) (layer "B.Cu") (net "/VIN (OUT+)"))
 (segment (start 5.437653 109.407553) (end 4.2 108.1699) (width 0.2) (layer "B.Cu") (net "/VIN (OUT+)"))
 (segment (start 20.58 103.6) (end 20.58 108.42) (width 0.2) (layer "B.Cu") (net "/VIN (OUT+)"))
 (segment (start 20.58 108.42) (end 19.592447 109.407553) (width 0.2) (layer "B.Cu") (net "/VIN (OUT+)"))
 (segment (start 27 126.6) (end 28.2 125.4) (width 0.2) (layer "B.Cu") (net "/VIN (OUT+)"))
 (segment (start 19.592447 109.407553) (end 5.437653 109.407553) (width 0.2) (layer "B.Cu") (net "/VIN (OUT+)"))
 (segment (start 27 127.2) (end 27 126.6) (width 0.2) (layer "B.Cu") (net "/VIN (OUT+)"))
 (segment (start 20.58 103.6) (end 20.4 103.78) (width 0.2) (layer "B.Cu") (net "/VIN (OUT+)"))
 (segment (start 3.66 42.54) (end 1.4 42.54) (width 0.2) (layer "F.Cu") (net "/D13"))
 (segment (start 4.4 41.8) (end 3.66 42.54) (width 0.2) (layer "F.Cu") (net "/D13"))
 (segment (start 4.4 13.6) (end 4.4 41.8) (width 0.2) (layer "F.Cu") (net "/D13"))
 (segment (start 4.5 13.5) (end 4.4 13.6) (width 0.2) (layer "F.Cu") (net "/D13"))
 (segment (start 13.85 13.5) (end 4.5 13.5) (width 0.2) (layer "F.Cu") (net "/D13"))
 (segment (start 22.4 52.8) (end 22.4 31) (width 0.2) (layer "B.Cu") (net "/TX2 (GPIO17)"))
 (segment (start 13.85 32.5) (end 13.85 33.5) (width 0.2) (layer "B.Cu") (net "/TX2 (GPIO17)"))
 (segment (start 28 52.8) (end 22.4 52.8) (width 0.2) (layer "B.Cu") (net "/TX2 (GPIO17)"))
 (segment (start 22.4 31) (end 15.35 31) (width 0.2) (layer "B.Cu") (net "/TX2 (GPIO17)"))
 (segment (start 15.35 31) (end 13.85 32.5) (width 0.2) (layer "B.Cu") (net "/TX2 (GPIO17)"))
 (segment (start 28.1 52.7) (end 28 52.8) (width 0.2) (layer "B.Cu") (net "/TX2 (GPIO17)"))
 (segment (start 15.1 80.8) (end 15.1 75.86) (width 0.2) (layer "B.Cu") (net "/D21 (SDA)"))
 (segment (start 15.1 75.86) (end 28.1 62.86) (width 0.2) (layer "B.Cu") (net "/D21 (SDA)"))
 (segment (start 17.6 80.8) (end 27.92 70.48) (width 0.2) (layer "B.Cu") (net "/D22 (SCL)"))
 (segment (start 27.92 70.48) (end 28.1 70.48) (width 0.2) (layer "B.Cu") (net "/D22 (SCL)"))
 (segment (start 6.8 103) (end 6.8 110.6) (width 0.2) (layer "F.Cu") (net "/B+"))
 (segment (start 6.75 110.65) (end 4.2 110.65) (width 0.2) (layer "F.Cu") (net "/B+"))
 (segment (start 6.8 110.6) (end 6.75 110.65) (width 0.2) (layer "F.Cu") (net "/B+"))
 (segment (start 3.8 103) (end 2 104.8) (width 0.2) (layer "F.Cu") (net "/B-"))
 (segment (start 2.25 119.65) (end 4.2 119.65) (width 0.2) (layer "F.Cu") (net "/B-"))
 (segment (start 2 119.4) (end 2.25 119.65) (width 0.2) (layer "F.Cu") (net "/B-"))
 (segment (start 2 104.8) (end 2 119.4) (width 0.2) (layer "F.Cu") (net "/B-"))
 (segment (start 4.26 103) (end 3.8 103) (width 0.2) (layer "F.Cu") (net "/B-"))
 (segment (start 23.6 122.2) (end 23.6 137.4) (width 0.2) (layer "F.Cu") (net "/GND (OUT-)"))
 (segment (start 23.6 137.4) (end 24.2 138) (width 0.2) (layer "F.Cu") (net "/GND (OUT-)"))
 (segment (start 24.2 138) (end 27 138) (width 0.2) (layer "F.Cu") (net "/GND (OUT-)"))
 (segment (start 4.2 122.15) (end 23.55 122.15) (width 0.2) (layer "F.Cu") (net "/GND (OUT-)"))
 (segment (start 23.55 122.15) (end 23.6 122.2) (width 0.2) (layer "F.Cu") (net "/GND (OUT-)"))
 (segment (start 5.4 41) (end 5.4 37.8) (width 0.2) (layer "F.Cu") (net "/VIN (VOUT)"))
 (segment (start 4.4 76.8) (end 5.4 75.8) (width 0.2) (layer "F.Cu") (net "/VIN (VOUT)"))
 (segment (start 5.4 75.8) (end 5.4 48.4) (width 0.2) (layer "F.Cu") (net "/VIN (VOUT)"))
 (segment (start 3.1 127.2) (end 1.6 125.7) (width 0.2) (layer "F.Cu") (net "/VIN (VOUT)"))
 (segment (start 1.6 125.7) (end 1.6 76.8) (width 0.2) (layer "F.Cu") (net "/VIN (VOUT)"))
 (segment (start 1.6 76.8) (end 4.4 76.8) (width 0.2) (layer "F.Cu") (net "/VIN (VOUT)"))
 (via (at 5.4 48.4) (size 0.6) (drill 0.3) (layers "F.Cu" "B.Cu") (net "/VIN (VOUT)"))
 (via (at 5.4 41) (size 0.6) (drill 0.3) (layers "F.Cu" "B.Cu") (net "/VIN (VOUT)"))
 (via (at 5.4 37.8) (size 0.6) (drill 0.3) (layers "F.Cu" "B.Cu") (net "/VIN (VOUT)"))
 (segment (start 5.4 48.4) (end 5.4 41) (width 0.2) (layer "B.Cu") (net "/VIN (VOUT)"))
 (segment (start 5.4 37.8) (end 5.06 37.46) (width 0.2) (layer "B.Cu") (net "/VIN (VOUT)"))
 (segment (start 5.06 37.46) (end 1.4 37.46) (width 0.2) (layer "B.Cu") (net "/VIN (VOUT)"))
 (segment (start 11.6 78.2) (end 23.2 78.2) (width 0.2) (layer "F.Cu") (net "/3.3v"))
 (segment (start 23.2 78.2) (end 23.2 51.4) (width 0.2) (layer "F.Cu") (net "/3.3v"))
 (via (at 23.2 51.4) (size 0.6) (drill 0.3) (layers "F.Cu" "B.Cu") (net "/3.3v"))
 (via (at 11.6 78.2) (size 0.6) (drill 0.3) (layers "F.Cu" "B.Cu") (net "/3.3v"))
 (segment (start 23.2 51.4) (end 23.2 37.4) (width 0.2) (layer "B.Cu") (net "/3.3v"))
 (segment (start 23.66 37.46) (end 28.1 37.46) (width 0.2) (layer "B.Cu") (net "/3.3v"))
 (segment (start 7.6 80.8) (end 7.6 78.2) (width 0.2) (layer "B.Cu") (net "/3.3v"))
 (segment (start 23.6 37.4) (end 23.66 37.46) (width 0.2) (layer "B.Cu") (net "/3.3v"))
 (segment (start 23.2 37.4) (end 23.6 37.4) (width 0.2) (layer "B.Cu") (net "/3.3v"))
 (segment (start 7.6 78.2) (end 11.6 78.2) (width 0.2) (layer "B.Cu") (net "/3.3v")))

